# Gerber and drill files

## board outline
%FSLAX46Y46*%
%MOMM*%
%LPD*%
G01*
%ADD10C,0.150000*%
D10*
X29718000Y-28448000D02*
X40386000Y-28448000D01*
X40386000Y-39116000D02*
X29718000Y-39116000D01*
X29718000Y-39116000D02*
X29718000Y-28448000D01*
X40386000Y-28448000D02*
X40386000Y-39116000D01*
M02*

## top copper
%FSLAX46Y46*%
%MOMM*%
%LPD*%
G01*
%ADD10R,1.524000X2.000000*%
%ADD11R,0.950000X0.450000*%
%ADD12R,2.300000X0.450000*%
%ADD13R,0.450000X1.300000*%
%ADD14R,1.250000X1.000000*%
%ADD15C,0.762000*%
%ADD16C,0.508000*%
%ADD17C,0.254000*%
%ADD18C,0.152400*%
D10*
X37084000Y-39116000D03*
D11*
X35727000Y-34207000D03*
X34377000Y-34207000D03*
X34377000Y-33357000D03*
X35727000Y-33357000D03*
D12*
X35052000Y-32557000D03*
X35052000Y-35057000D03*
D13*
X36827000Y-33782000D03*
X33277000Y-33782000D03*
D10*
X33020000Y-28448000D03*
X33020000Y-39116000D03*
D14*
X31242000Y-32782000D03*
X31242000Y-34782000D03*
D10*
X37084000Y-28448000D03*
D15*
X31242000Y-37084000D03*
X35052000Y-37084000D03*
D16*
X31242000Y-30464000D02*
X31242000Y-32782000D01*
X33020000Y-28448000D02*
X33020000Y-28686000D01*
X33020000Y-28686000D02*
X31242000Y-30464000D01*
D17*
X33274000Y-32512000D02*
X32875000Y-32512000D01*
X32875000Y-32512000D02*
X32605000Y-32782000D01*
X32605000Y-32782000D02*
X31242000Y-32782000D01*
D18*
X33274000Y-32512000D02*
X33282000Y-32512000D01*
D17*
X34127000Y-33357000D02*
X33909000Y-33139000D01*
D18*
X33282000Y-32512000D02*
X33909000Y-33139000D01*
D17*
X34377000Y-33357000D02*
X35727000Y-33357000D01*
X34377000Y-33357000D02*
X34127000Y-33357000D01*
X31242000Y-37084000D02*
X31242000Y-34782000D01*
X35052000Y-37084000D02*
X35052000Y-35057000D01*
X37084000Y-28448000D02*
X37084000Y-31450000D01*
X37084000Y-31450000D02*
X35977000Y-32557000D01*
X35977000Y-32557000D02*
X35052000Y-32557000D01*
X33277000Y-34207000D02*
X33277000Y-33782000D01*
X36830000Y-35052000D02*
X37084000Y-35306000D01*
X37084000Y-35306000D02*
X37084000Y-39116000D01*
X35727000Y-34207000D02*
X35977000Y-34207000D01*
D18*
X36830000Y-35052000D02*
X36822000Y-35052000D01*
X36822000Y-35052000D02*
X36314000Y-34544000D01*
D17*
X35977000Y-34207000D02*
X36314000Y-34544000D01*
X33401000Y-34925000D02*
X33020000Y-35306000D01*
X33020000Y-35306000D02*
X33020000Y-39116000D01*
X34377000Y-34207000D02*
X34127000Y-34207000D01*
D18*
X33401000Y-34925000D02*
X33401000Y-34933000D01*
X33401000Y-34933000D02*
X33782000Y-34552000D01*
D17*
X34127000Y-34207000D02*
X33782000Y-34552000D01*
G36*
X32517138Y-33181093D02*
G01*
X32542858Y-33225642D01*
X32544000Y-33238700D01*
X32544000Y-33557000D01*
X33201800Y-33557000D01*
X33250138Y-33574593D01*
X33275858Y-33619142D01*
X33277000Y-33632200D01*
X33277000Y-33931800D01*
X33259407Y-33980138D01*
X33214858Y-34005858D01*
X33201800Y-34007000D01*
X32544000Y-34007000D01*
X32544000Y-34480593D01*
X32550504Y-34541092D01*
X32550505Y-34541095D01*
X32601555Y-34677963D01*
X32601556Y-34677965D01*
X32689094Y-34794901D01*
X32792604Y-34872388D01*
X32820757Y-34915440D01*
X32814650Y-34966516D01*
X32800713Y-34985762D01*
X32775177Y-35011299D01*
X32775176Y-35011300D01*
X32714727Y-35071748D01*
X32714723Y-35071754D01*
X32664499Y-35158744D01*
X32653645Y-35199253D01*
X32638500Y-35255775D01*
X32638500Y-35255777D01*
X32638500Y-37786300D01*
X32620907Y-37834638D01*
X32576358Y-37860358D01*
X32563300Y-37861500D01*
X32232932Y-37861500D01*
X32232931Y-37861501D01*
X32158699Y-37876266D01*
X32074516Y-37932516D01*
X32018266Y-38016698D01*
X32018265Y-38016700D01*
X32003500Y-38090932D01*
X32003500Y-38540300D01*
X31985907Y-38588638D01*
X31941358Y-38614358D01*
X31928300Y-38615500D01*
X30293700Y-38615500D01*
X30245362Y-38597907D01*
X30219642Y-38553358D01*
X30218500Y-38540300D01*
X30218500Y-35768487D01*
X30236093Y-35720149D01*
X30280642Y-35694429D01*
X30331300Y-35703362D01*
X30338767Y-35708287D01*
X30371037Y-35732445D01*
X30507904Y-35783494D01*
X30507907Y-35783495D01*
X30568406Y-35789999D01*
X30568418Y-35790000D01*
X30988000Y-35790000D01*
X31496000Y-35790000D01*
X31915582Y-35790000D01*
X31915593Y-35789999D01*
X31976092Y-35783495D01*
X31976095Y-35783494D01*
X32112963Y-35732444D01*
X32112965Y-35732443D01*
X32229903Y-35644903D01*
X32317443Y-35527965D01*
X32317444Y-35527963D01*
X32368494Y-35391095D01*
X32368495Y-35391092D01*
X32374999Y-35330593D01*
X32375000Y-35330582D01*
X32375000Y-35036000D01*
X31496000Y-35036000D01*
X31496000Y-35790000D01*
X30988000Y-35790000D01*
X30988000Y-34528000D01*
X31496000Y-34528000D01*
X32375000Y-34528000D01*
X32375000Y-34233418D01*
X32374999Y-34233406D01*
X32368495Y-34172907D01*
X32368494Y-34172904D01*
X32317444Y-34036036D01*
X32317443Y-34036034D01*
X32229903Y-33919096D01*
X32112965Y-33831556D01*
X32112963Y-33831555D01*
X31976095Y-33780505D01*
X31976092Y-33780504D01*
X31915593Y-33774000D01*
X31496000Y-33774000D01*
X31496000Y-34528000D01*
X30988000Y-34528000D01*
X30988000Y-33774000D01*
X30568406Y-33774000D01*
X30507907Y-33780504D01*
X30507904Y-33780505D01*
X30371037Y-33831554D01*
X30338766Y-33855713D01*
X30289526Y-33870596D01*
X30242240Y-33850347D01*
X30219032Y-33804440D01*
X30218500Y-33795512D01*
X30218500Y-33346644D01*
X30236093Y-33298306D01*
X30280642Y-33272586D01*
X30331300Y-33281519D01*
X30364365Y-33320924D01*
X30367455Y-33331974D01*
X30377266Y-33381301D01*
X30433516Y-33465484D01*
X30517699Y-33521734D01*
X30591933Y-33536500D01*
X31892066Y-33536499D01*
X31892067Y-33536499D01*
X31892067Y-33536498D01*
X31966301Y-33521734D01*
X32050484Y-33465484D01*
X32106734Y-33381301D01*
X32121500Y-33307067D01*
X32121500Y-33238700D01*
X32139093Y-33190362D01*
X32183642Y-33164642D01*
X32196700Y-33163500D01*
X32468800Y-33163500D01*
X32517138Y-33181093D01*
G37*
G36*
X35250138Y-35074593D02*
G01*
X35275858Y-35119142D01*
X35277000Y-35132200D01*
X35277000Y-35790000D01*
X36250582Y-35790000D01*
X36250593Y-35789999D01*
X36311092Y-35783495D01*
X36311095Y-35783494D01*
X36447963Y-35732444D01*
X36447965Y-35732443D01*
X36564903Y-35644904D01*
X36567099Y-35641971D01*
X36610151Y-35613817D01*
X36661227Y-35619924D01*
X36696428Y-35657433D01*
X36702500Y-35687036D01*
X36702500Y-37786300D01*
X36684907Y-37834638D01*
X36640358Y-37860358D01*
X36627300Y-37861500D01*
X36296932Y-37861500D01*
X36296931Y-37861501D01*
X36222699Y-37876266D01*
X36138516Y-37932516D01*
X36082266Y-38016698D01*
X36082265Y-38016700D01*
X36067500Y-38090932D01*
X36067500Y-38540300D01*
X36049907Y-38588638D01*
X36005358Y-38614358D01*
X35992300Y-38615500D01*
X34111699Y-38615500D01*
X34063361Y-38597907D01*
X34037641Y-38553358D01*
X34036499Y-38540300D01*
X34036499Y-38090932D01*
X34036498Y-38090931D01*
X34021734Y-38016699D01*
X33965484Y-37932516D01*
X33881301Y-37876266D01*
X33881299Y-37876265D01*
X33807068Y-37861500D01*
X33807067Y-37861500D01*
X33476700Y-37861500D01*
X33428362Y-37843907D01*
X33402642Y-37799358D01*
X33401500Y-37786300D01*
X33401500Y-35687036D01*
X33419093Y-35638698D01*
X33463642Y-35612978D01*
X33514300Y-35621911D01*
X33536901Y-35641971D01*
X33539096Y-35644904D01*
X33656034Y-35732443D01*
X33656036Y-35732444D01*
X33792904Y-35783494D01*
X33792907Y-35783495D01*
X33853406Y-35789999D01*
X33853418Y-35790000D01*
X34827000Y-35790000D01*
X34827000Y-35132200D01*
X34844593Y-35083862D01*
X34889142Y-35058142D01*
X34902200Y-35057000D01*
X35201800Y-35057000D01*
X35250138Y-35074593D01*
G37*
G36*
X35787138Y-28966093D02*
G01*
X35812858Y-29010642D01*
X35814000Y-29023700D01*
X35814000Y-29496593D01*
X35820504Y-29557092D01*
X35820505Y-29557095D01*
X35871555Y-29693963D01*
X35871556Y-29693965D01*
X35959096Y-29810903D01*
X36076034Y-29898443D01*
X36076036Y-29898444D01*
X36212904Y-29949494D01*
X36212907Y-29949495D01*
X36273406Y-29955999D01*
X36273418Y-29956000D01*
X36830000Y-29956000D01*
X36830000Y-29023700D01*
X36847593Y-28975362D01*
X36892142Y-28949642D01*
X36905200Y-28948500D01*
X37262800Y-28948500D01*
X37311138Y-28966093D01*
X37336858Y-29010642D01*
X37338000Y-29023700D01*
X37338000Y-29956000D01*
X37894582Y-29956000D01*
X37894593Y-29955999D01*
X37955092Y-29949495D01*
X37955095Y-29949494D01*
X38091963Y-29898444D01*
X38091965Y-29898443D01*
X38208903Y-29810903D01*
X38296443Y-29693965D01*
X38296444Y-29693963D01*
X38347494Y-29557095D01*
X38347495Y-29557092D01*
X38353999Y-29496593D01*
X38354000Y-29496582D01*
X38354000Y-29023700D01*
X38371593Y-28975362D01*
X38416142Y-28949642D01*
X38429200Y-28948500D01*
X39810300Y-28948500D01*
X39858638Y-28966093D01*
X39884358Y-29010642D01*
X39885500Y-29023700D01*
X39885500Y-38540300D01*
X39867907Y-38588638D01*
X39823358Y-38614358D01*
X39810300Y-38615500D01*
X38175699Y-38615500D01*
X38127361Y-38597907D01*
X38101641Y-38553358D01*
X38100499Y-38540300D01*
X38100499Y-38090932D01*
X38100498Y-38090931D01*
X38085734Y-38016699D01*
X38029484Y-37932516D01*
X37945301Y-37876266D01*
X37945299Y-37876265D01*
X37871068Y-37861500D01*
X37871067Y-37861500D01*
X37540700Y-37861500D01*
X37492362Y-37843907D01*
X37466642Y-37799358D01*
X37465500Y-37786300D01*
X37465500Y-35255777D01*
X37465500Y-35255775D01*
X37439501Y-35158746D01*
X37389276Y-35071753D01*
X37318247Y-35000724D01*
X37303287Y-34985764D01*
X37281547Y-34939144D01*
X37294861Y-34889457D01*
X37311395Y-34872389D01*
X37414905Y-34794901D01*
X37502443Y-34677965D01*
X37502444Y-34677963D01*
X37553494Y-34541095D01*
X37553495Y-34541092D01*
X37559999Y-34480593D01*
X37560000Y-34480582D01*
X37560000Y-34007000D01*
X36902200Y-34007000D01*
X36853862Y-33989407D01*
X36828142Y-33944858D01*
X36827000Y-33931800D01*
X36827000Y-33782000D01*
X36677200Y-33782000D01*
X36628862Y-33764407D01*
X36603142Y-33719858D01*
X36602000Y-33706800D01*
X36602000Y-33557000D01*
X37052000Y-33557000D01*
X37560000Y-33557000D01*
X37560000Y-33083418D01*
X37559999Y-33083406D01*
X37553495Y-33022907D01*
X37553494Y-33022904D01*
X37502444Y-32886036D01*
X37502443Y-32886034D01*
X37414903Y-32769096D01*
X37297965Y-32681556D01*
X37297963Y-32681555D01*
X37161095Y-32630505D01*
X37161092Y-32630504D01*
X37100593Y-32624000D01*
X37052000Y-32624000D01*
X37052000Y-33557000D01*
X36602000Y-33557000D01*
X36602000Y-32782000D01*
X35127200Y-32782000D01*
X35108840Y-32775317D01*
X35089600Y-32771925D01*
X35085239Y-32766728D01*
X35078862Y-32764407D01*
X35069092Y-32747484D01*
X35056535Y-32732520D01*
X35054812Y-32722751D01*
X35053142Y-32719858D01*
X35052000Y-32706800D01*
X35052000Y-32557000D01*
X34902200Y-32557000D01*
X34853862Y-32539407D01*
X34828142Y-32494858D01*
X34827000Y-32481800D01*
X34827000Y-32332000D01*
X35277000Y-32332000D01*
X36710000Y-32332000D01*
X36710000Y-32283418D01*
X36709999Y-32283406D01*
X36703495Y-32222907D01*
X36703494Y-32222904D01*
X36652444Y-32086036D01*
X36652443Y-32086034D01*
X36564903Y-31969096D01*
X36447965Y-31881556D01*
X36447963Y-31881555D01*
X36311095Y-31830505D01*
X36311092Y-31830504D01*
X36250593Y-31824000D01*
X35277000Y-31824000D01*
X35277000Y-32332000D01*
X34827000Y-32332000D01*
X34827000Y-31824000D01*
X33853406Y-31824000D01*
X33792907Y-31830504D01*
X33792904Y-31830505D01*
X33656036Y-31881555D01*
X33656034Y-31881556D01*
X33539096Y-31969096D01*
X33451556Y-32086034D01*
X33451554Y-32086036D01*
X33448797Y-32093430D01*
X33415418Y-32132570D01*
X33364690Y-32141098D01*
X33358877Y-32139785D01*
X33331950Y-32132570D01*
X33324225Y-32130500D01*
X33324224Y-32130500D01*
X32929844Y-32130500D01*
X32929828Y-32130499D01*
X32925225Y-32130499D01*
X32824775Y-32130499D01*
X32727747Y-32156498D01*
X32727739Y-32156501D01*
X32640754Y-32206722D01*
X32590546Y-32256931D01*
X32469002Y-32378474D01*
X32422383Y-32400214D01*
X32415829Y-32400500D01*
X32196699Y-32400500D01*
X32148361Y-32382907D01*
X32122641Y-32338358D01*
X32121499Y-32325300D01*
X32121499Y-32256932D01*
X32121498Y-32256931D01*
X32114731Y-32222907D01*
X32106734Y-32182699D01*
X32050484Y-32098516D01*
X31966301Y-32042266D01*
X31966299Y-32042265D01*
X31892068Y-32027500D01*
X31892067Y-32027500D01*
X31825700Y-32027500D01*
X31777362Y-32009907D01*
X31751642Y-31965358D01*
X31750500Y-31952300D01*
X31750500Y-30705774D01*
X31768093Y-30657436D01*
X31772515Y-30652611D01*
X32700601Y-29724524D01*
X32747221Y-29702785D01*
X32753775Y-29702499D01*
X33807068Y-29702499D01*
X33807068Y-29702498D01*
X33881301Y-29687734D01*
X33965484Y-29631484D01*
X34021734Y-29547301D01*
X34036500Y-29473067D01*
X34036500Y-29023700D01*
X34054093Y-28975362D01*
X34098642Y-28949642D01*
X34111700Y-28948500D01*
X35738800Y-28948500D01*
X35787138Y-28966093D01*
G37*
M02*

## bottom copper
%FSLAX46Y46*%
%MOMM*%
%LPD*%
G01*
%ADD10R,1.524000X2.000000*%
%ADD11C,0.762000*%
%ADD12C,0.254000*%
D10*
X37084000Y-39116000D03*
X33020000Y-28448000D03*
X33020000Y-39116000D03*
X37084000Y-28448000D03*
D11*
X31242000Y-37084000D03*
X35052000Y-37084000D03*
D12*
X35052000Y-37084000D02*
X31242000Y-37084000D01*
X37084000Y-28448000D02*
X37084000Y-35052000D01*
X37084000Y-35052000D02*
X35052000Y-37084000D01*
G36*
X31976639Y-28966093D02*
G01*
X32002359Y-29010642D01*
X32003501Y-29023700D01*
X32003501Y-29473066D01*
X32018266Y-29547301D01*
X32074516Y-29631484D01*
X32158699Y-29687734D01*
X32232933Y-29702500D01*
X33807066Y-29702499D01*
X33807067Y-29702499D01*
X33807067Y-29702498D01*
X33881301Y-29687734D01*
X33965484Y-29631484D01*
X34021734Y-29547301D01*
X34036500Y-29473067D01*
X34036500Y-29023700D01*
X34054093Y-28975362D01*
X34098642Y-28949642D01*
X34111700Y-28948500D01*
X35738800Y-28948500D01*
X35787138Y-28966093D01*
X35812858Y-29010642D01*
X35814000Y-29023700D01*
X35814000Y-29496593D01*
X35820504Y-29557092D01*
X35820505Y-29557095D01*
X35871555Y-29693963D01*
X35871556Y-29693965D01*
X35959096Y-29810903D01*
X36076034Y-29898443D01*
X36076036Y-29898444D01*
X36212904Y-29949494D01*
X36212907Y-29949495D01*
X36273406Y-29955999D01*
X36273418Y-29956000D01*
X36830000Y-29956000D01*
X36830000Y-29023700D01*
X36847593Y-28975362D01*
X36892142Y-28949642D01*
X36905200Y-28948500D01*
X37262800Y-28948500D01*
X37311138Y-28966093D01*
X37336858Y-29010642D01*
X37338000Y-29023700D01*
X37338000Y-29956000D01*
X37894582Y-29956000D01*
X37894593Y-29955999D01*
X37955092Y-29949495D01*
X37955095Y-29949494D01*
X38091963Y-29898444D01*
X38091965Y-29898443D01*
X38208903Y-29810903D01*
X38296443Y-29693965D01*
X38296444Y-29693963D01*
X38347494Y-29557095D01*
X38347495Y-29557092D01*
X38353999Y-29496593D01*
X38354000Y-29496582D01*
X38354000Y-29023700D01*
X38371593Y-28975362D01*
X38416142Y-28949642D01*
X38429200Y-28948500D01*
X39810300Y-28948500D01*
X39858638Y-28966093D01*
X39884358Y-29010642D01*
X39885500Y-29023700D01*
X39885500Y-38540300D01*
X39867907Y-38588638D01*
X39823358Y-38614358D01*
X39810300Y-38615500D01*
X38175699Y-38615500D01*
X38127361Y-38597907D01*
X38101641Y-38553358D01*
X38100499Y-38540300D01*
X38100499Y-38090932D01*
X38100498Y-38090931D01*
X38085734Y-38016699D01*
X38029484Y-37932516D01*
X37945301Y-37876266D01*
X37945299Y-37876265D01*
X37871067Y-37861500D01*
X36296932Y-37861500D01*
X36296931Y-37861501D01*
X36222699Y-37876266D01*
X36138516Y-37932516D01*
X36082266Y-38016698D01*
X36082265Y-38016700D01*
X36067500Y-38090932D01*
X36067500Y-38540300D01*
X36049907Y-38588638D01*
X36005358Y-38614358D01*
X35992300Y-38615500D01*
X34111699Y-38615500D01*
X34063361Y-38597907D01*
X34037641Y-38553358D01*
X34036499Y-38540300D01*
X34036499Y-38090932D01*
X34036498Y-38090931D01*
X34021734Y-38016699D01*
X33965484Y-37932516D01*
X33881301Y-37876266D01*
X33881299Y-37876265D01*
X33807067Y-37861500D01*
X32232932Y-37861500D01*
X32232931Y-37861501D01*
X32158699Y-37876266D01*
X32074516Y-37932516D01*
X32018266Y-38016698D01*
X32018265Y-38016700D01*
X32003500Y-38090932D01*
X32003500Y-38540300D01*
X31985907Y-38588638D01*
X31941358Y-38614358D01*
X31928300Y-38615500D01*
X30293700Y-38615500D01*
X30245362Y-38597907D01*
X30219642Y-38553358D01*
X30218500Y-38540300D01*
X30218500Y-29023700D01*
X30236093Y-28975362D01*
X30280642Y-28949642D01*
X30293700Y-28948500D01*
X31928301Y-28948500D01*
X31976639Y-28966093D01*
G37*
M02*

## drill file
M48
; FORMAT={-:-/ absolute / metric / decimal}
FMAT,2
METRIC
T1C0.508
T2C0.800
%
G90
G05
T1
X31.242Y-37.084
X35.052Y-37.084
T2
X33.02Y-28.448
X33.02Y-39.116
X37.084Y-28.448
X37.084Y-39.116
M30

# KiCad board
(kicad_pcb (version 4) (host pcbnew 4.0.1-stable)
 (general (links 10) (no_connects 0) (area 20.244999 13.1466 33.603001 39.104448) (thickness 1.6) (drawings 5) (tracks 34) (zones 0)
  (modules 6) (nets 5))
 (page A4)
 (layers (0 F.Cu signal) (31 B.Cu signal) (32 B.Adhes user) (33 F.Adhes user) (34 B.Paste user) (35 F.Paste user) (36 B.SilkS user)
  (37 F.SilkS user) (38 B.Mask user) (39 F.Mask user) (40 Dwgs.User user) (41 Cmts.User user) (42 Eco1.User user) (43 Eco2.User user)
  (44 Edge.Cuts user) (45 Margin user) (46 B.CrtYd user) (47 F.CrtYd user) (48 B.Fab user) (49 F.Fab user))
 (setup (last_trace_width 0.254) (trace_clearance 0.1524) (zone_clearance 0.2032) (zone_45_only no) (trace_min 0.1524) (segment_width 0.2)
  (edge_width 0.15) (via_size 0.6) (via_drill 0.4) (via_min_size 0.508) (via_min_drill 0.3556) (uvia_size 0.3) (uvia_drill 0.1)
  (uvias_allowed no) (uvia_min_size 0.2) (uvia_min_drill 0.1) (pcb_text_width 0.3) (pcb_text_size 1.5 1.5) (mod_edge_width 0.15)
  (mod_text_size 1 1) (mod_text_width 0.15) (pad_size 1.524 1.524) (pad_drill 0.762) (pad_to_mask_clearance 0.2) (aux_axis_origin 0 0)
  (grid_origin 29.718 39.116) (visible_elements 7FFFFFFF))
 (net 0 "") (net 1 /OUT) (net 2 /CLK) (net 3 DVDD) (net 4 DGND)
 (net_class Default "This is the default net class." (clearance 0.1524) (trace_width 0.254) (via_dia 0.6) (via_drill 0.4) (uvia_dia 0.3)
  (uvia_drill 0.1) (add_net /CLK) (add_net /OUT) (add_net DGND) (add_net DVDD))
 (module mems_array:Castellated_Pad (layer F.Cu) (at 37.084 39.116)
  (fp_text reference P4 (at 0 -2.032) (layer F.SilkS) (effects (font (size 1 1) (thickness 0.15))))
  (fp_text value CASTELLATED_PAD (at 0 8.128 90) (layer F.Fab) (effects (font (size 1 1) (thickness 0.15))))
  (pad 1 thru_hole rect (at 0 0) (size 1.524 2) (drill 0.8) (layers *.Cu *.Mask F.SilkS) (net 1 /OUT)))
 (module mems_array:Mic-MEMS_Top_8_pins (layer F.Cu) (at 35.052 33.782 90)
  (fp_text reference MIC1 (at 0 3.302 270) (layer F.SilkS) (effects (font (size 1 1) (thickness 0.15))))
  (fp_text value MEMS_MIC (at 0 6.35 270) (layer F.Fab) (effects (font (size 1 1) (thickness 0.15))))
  (pad 4 smd rect (at -0.425 0.675 90) (size 0.45 0.95) (layers F.Cu F.Paste F.Mask) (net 1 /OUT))
  (pad 3 smd rect (at -0.425 -0.675 90) (size 0.45 0.95) (layers F.Cu F.Paste F.Mask) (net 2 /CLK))
  (pad 2 smd rect (at 0.425 -0.675 90) (size 0.45 0.95) (layers F.Cu F.Paste F.Mask) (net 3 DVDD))
  (pad 1 smd rect (at 0.425 0.675 90) (size 0.45 0.95) (layers F.Cu F.Paste F.Mask) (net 3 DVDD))
  (pad 5 smd rect (at 1.225 0 90) (size 0.45 2.3) (layers F.Cu F.Paste F.Mask) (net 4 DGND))
  (pad 5 smd rect (at -1.275 0 90) (size 0.45 2.3) (layers F.Cu F.Paste F.Mask) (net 4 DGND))
  (pad 5 smd rect (at 0 1.775 90) (size 1.3 0.45) (layers F.Cu F.Paste F.Mask) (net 4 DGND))
  (pad 5 smd rect (at 0 -1.775 90) (size 1.3 0.45) (layers F.Cu F.Paste F.Mask) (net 4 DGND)))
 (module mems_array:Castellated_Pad (layer F.Cu) (at 33.02 28.448)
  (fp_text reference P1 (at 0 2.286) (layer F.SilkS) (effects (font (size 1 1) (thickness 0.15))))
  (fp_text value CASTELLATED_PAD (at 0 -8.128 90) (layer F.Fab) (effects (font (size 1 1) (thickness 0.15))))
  (pad 1 thru_hole rect (at 0 0) (size 1.524 2) (drill 0.8) (layers *.Cu *.Mask F.SilkS) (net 3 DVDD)))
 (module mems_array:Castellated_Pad (layer F.Cu) (at 33.02 39.116)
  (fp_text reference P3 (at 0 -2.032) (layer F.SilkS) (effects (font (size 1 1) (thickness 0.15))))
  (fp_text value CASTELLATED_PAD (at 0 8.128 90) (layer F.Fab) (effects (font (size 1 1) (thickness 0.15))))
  (pad 1 thru_hole rect (at 0 0) (size 1.524 2) (drill 0.8) (layers *.Cu *.Mask F.SilkS) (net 2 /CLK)))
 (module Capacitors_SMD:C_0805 (layer F.Cu) (at 31.242 33.782 270)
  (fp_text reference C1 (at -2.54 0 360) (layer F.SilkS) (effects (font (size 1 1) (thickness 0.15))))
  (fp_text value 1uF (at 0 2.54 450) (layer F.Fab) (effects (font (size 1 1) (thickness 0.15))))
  (pad 1 smd rect (at -1 0 270) (size 1 1.25) (layers F.Cu F.Paste F.Mask) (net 3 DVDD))
  (pad 2 smd rect (at 1 0 270) (size 1 1.25) (layers F.Cu F.Paste F.Mask) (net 4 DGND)))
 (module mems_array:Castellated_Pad (layer F.Cu) (at 37.084 28.448)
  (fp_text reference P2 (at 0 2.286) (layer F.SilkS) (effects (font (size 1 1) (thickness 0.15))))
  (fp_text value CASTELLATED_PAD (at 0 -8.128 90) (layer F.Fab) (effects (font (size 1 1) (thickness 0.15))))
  (pad 1 thru_hole rect (at 0 0) (size 1.524 2) (drill 0.8) (layers *.Cu *.Mask F.SilkS) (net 4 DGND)))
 (gr_line (start 29.718 28.448) (end 40.386 28.448) (layer Edge.Cuts) (width 0.15))
 (gr_line (start 40.386 39.116) (end 29.718 39.116) (layer Edge.Cuts) (width 0.15))
 (gr_line (start 29.718 39.116) (end 29.718 28.448) (layer Edge.Cuts) (width 0.15))
 (gr_line (start 40.386 28.448) (end 40.386 39.116) (layer Edge.Cuts) (width 0.15))
 (segment (start 31.242 30.464) (end 31.242 32.782) (width 0.508) (layer F.Cu) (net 3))
 (segment (start 33.02 28.448) (end 33.02 28.686) (width 0.508) (layer F.Cu) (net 3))
 (segment (start 33.02 28.686) (end 31.242 30.464) (width 0.508) (layer F.Cu) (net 3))
 (segment (start 33.274 32.512) (end 32.875 32.512) (width 0.254) (layer F.Cu) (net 3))
 (segment (start 32.875 32.512) (end 32.605 32.782) (width 0.254) (layer F.Cu) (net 3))
 (segment (start 32.605 32.782) (end 31.242 32.782) (width 0.254) (layer F.Cu) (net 3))
 (segment (start 33.274 32.512) (end 33.282 32.512) (width 0.1524) (layer F.Cu) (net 3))
 (segment (start 34.127 33.357) (end 33.909 33.139) (width 0.254) (layer F.Cu) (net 3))
 (segment (start 33.282 32.512) (end 33.909 33.139) (width 0.1524) (layer F.Cu) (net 3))
 (segment (start 34.377 33.357) (end 35.727 33.357) (width 0.254) (layer F.Cu) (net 3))
 (segment (start 34.377 33.357) (end 34.127 33.357) (width 0.254) (layer F.Cu) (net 3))
 (segment (start 31.242 37.084) (end 31.242 34.782) (width 0.254) (layer F.Cu) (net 4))
 (segment (start 35.052 37.084) (end 31.242 37.084) (width 0.254) (layer B.Cu) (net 4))
 (via (at 31.242 37.084) (size 0.762) (drill 0.508) (layers F.Cu B.Cu) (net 4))
 (segment (start 35.052 37.084) (end 35.052 35.057) (width 0.254) (layer F.Cu) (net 4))
 (segment (start 37.084 28.448) (end 37.084 35.052) (width 0.254) (layer B.Cu) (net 4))
 (segment (start 37.084 35.052) (end 35.052 37.084) (width 0.254) (layer B.Cu) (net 4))
 (via (at 35.052 37.084) (size 0.762) (drill 0.508) (layers F.Cu B.Cu) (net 4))
 (segment (start 37.084 28.448) (end 37.084 31.45) (width 0.254) (layer F.Cu) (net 4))
 (segment (start 37.084 31.45) (end 35.977 32.557) (width 0.254) (layer F.Cu) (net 4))
 (segment (start 35.977 32.557) (end 35.052 32.557) (width 0.254) (layer F.Cu) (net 4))
 (segment (start 33.277 34.207) (end 33.277 33.782) (width 0.254) (layer F.Cu) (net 4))
 (segment (start 36.83 35.052) (end 37.084 35.306) (width 0.254) (layer F.Cu) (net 1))
 (segment (start 37.084 35.306) (end 37.084 39.116) (width 0.254) (layer F.Cu) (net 1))
 (segment (start 35.727 34.207) (end 35.977 34.207) (width 0.254) (layer F.Cu) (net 1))
 (segment (start 36.83 35.052) (end 36.822 35.052) (width 0.1524) (layer F.Cu) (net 1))
 (segment (start 36.822 35.052) (end 36.314 34.544) (width 0.1524) (layer F.Cu) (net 1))
 (segment (start 35.977 34.207) (end 36.314 34.544) (width 0.254) (layer F.Cu) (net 1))
 (segment (start 33.401 34.925) (end 33.02 35.306) (width 0.254) (layer F.Cu) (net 2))
 (segment (start 33.02 35.306) (end 33.02 39.116) (width 0.254) (layer F.Cu) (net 2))
 (segment (start 34.377 34.207) (end 34.127 34.207) (width 0.254) (layer F.Cu) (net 2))
 (segment (start 33.401 34.925) (end 33.401 34.933) (width 0.1524) (layer F.Cu) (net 2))
 (segment (start 33.401 34.933) (end 33.782 34.552) (width 0.1524) (layer F.Cu) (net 2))
 (segment (start 34.127 34.207) (end 33.782 34.552) (width 0.254) (layer F.Cu) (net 2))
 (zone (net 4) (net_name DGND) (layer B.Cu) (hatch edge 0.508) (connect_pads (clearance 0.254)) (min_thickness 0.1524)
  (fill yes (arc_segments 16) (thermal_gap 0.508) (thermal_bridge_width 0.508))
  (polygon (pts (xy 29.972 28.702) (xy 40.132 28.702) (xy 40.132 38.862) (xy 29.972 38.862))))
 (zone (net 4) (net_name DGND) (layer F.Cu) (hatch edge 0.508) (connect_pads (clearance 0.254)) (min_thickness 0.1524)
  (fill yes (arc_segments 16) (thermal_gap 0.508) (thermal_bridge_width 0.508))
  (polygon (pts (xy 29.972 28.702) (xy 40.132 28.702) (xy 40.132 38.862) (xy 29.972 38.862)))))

